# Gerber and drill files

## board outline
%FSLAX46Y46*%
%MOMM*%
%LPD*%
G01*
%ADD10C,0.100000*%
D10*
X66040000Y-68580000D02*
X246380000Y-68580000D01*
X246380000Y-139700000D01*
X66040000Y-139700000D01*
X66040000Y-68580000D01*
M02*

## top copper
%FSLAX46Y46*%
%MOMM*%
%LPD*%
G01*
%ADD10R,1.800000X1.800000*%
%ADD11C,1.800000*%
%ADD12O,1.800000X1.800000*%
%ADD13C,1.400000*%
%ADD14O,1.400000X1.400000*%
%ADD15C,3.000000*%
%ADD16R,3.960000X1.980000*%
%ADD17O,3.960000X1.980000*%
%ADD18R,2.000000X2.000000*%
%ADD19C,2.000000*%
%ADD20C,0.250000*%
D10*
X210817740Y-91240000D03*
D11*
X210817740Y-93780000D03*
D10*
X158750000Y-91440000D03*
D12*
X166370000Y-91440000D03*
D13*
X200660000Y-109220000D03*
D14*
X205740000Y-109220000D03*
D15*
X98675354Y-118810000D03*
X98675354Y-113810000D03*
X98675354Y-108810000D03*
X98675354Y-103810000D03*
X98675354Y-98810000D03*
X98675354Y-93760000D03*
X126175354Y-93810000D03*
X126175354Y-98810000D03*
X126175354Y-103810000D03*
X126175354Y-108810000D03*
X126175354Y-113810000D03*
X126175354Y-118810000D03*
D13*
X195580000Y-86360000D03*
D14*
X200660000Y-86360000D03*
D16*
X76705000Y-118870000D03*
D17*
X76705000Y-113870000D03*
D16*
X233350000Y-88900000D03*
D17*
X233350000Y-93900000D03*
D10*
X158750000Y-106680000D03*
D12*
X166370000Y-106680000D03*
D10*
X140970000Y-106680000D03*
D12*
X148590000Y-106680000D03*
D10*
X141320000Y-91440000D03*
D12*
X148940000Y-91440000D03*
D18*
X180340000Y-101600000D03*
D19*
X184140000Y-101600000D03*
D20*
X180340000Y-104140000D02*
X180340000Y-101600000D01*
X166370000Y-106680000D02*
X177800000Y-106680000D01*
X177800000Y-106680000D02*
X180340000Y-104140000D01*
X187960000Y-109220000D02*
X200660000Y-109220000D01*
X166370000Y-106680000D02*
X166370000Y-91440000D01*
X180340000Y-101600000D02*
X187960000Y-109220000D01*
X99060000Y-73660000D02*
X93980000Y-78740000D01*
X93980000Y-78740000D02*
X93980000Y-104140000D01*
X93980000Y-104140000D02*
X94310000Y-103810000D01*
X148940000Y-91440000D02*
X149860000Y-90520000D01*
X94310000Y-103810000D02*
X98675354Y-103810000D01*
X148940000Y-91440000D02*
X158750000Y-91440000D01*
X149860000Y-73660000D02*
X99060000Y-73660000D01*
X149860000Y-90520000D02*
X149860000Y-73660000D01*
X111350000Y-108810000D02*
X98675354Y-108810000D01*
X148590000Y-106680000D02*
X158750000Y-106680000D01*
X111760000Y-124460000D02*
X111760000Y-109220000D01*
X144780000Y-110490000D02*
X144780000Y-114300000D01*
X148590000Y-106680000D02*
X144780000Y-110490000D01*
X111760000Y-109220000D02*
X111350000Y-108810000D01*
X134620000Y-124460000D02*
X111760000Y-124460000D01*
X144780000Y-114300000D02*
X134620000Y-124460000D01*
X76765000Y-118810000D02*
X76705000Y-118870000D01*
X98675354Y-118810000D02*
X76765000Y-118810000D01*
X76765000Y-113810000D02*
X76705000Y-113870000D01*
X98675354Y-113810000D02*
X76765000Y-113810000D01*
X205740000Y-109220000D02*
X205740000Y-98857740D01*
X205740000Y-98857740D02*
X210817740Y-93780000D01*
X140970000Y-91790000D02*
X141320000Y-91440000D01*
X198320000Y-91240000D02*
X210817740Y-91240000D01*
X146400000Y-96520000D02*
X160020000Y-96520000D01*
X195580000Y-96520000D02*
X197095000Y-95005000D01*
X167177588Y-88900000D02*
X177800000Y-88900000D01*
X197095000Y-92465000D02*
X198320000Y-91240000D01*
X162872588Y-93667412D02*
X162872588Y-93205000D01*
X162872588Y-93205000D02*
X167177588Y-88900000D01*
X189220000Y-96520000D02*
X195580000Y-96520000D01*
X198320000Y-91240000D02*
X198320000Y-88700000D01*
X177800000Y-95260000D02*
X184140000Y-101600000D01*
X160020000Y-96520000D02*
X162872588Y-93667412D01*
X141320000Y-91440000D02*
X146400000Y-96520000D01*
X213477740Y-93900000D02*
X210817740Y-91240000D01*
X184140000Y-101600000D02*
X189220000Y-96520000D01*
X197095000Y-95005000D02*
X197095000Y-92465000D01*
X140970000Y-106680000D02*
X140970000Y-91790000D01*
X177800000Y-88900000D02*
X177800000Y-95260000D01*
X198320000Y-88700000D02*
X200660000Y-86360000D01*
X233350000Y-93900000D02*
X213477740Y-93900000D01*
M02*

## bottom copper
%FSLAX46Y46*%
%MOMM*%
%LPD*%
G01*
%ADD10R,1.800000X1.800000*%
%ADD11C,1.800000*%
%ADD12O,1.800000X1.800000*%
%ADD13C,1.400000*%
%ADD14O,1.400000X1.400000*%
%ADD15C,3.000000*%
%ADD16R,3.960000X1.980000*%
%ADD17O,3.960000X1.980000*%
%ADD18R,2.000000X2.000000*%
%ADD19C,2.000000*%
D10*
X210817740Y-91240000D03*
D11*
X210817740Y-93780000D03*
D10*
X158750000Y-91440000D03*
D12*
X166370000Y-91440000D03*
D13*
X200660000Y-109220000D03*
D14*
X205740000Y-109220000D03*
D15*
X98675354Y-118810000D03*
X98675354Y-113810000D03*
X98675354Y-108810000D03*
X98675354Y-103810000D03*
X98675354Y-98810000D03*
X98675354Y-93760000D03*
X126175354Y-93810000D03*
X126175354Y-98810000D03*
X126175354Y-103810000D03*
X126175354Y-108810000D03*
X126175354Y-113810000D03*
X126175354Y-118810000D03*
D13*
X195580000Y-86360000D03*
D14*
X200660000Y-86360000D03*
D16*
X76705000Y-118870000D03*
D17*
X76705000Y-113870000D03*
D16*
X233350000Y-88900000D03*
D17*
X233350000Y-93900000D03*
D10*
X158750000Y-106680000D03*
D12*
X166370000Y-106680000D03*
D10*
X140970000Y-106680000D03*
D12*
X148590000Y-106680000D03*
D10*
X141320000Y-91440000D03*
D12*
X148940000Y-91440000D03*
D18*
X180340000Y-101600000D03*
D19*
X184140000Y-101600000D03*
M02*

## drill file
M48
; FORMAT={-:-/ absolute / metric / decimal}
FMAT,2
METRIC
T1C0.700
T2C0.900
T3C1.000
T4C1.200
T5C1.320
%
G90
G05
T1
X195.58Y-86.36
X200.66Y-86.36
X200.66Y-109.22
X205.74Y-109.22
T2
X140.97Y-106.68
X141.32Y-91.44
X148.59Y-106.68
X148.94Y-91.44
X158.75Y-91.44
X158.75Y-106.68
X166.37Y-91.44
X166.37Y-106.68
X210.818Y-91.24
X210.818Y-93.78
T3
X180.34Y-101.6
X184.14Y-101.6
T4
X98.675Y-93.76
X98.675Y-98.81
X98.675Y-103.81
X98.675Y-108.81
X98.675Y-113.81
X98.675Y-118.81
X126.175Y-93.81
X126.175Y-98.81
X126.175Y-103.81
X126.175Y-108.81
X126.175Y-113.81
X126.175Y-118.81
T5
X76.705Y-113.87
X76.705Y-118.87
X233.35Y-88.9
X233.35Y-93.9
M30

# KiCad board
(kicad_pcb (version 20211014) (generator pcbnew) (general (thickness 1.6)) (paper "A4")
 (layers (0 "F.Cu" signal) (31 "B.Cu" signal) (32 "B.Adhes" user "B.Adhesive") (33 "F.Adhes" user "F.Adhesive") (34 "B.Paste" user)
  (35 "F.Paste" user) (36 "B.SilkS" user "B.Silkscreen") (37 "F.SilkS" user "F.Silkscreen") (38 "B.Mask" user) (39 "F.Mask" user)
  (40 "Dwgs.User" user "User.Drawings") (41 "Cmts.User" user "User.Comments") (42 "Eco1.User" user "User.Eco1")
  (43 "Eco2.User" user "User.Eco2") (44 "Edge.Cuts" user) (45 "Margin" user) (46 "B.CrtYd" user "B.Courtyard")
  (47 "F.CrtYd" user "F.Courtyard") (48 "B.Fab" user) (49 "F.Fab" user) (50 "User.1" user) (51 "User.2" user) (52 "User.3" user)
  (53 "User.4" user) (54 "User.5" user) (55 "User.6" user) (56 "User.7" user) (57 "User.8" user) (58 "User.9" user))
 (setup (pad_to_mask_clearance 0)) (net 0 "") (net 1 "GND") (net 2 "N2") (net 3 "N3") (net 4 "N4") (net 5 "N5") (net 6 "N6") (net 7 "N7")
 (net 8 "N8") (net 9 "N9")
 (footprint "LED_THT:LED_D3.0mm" (layer "F.Cu") (at 210.81774 91.24 -90)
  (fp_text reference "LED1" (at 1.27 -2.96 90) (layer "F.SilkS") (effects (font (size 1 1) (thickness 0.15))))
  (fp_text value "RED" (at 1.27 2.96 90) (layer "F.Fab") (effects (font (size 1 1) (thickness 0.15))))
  (pad "1" thru_hole rect (at 0 0 270) (size 1.8 1.8) (drill 0.9) (layers *.Cu *.Mask) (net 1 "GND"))
  (pad "2" thru_hole circle (at 2.54 0 270) (size 1.8 1.8) (drill 0.9) (layers *.Cu *.Mask) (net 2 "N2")))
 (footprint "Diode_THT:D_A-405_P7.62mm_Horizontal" (layer "F.Cu") (at 158.75 91.44)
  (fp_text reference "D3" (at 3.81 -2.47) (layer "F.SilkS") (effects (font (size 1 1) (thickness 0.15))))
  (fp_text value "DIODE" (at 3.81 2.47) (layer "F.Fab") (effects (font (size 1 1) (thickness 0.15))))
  (pad "1" thru_hole rect (at 0 0) (size 1.8 1.8) (drill 0.9) (layers *.Cu *.Mask) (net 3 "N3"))
  (pad "2" thru_hole oval (at 7.62 0) (size 1.8 1.8) (drill 0.9) (layers *.Cu *.Mask) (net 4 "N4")))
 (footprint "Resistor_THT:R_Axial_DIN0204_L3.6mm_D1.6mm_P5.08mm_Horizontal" (layer "F.Cu") (at 200.66 109.22)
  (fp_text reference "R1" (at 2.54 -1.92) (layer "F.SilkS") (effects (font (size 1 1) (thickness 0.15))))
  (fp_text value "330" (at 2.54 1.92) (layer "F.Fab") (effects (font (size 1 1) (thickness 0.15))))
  (pad "1" thru_hole circle (at 0 0) (size 1.4 1.4) (drill 0.7) (layers *.Cu *.Mask) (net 4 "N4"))
  (pad "2" thru_hole oval (at 5.08 0) (size 1.4 1.4) (drill 0.7) (layers *.Cu *.Mask) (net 2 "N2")))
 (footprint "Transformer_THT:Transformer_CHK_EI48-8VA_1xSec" (layer "F.Cu") (at 98.675354 118.81)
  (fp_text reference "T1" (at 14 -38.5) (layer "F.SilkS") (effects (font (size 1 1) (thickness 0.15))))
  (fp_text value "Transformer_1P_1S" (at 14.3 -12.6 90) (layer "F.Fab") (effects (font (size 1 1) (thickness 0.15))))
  (pad "1" thru_hole circle (at 0 0) (size 3 3) (drill 1.2) (layers *.Cu *.Mask) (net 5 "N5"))
  (pad "2" thru_hole circle (at 0 -5) (size 3 3) (drill 1.2) (layers *.Cu *.Mask) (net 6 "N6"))
  (pad "3" thru_hole circle (at 0 -10) (size 3 3) (drill 1.2) (layers *.Cu *.Mask) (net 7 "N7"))
  (pad "4" thru_hole circle (at 0 -15) (size 3 3) (drill 1.2) (layers *.Cu *.Mask) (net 3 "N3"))
  (pad "5" thru_hole circle (at 0 -20) (size 3 3) (drill 1.2) (layers *.Cu *.Mask))
  (pad "6" thru_hole circle (at 0 -25.05) (size 3 3) (drill 1.2) (layers *.Cu *.Mask))
  (pad "7" thru_hole circle (at 27.5 -25) (size 3 3) (drill 1.2) (layers *.Cu *.Mask))
  (pad "8" thru_hole circle (at 27.5 -20) (size 3 3) (drill 1.2) (layers *.Cu *.Mask))
  (pad "9" thru_hole circle (at 27.5 -15) (size 3 3) (drill 1.2) (layers *.Cu *.Mask))
  (pad "10" thru_hole circle (at 27.5 -10) (size 3 3) (drill 1.2) (layers *.Cu *.Mask))
  (pad "11" thru_hole circle (at 27.5 -5) (size 3 3) (drill 1.2) (layers *.Cu *.Mask))
  (pad "12" thru_hole circle (at 27.5 0) (size 3 3) (drill 1.2) (layers *.Cu *.Mask)))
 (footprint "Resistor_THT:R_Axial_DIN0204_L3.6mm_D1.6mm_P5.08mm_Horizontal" (layer "F.Cu") (at 195.58 86.36)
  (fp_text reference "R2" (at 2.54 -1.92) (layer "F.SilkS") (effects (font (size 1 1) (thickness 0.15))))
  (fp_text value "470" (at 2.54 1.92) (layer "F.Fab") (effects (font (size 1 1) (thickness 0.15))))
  (pad "1" thru_hole circle (at 0 0) (size 1.4 1.4) (drill 0.7) (layers *.Cu *.Mask) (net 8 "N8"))
  (pad "2" thru_hole oval (at 5.08 0) (size 1.4 1.4) (drill 0.7) (layers *.Cu *.Mask) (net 1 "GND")))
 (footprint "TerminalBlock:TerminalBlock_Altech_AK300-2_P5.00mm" (layer "F.Cu") (at 76.705 118.87 90)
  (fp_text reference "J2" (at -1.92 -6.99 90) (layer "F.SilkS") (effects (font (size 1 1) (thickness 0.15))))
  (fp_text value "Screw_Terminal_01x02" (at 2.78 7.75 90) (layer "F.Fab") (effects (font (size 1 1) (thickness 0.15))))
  (pad "1" thru_hole rect (at 0 0 90) (size 1.98 3.96) (drill 1.32) (layers *.Cu *.Mask) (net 5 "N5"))
  (pad "2" thru_hole oval (at 5 0 90) (size 1.98 3.96) (drill 1.32) (layers *.Cu *.Mask) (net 6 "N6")))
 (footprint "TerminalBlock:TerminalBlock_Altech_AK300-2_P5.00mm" (layer "F.Cu") (at 233.35 88.9 -90)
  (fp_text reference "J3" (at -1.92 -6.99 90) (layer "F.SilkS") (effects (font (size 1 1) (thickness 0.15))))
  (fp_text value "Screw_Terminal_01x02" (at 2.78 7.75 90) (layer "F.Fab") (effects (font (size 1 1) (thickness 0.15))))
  (pad "1" thru_hole rect (at 0 0 270) (size 1.98 3.96) (drill 1.32) (layers *.Cu *.Mask) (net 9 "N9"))
  (pad "2" thru_hole oval (at 5 0 270) (size 1.98 3.96) (drill 1.32) (layers *.Cu *.Mask) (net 1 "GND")))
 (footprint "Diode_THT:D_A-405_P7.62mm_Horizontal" (layer "F.Cu") (at 158.75 106.68)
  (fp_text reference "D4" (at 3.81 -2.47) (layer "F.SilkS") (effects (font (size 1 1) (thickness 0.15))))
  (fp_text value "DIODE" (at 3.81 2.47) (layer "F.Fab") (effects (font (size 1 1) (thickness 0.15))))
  (pad "1" thru_hole rect (at 0 0) (size 1.8 1.8) (drill 0.9) (layers *.Cu *.Mask) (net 7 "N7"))
  (pad "2" thru_hole oval (at 7.62 0) (size 1.8 1.8) (drill 0.9) (layers *.Cu *.Mask) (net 4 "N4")))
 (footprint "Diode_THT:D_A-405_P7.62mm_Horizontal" (layer "F.Cu") (at 140.97 106.68)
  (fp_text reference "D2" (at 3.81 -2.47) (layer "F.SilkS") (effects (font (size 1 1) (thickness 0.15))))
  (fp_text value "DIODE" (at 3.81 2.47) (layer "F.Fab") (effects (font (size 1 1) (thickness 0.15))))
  (pad "1" thru_hole rect (at 0 0) (size 1.8 1.8) (drill 0.9) (layers *.Cu *.Mask) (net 1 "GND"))
  (pad "2" thru_hole oval (at 7.62 0) (size 1.8 1.8) (drill 0.9) (layers *.Cu *.Mask) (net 7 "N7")))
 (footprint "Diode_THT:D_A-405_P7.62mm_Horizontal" (layer "F.Cu") (at 141.32 91.44)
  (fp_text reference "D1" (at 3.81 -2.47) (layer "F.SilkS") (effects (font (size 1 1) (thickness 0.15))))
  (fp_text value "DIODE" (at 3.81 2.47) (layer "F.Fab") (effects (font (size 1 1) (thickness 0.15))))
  (pad "1" thru_hole rect (at 0 0) (size 1.8 1.8) (drill 0.9) (layers *.Cu *.Mask) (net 1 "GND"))
  (pad "2" thru_hole oval (at 7.62 0) (size 1.8 1.8) (drill 0.9) (layers *.Cu *.Mask) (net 3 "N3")))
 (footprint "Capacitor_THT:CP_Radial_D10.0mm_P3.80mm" (layer "F.Cu") (at 180.34 101.6)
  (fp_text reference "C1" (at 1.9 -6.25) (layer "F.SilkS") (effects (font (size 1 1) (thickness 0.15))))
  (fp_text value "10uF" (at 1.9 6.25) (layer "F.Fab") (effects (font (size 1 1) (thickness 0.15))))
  (pad "1" thru_hole rect (at 0 0) (size 2 2) (drill 1) (layers *.Cu *.Mask) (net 4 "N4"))
  (pad "2" thru_hole circle (at 3.8 0) (size 2 2) (drill 1) (layers *.Cu *.Mask) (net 1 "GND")))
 (gr_rect (start 66.04 68.58) (end 246.38 139.7) (layer "Edge.Cuts") (width 0.1) (fill none))
 (segment (start 180.34 104.14) (end 180.34 101.6) (width 0.25) (layer "F.Cu") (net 4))
 (segment (start 166.37 106.68) (end 177.8 106.68) (width 0.25) (layer "F.Cu") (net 4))
 (segment (start 177.8 106.68) (end 180.34 104.14) (width 0.25) (layer "F.Cu") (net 4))
 (segment (start 187.96 109.22) (end 200.66 109.22) (width 0.25) (layer "F.Cu") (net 4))
 (segment (start 166.37 106.68) (end 166.37 91.44) (width 0.25) (layer "F.Cu") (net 4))
 (segment (start 180.34 101.6) (end 187.96 109.22) (width 0.25) (layer "F.Cu") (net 4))
 (segment (start 99.06 73.66) (end 93.98 78.74) (width 0.25) (layer "F.Cu") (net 3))
 (segment (start 93.98 78.74) (end 93.98 104.14) (width 0.25) (layer "F.Cu") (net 3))
 (segment (start 93.98 104.14) (end 94.31 103.81) (width 0.25) (layer "F.Cu") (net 3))
 (segment (start 148.94 91.44) (end 149.86 90.52) (width 0.25) (layer "F.Cu") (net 3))
 (segment (start 94.31 103.81) (end 98.675354 103.81) (width 0.25) (layer "F.Cu") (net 3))
 (segment (start 148.94 91.44) (end 158.75 91.44) (width 0.25) (layer "F.Cu") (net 3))
 (segment (start 149.86 73.66) (end 99.06 73.66) (width 0.25) (layer "F.Cu") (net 3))
 (segment (start 149.86 90.52) (end 149.86 73.66) (width 0.25) (layer "F.Cu") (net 3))
 (segment (start 111.35 108.81) (end 98.675354 108.81) (width 0.25) (layer "F.Cu") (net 7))
 (segment (start 148.59 106.68) (end 158.75 106.68) (width 0.25) (layer "F.Cu") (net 7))
 (segment (start 111.76 124.46) (end 111.76 109.22) (width 0.25) (layer "F.Cu") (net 7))
 (segment (start 144.78 110.49) (end 144.78 114.3) (width 0.25) (layer "F.Cu") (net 7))
 (segment (start 148.59 106.68) (end 144.78 110.49) (width 0.25) (layer "F.Cu") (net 7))
 (segment (start 111.76 109.22) (end 111.35 108.81) (width 0.25) (layer "F.Cu") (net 7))
 (segment (start 134.62 124.46) (end 111.76 124.46) (width 0.25) (layer "F.Cu") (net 7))
 (segment (start 144.78 114.3) (end 134.62 124.46) (width 0.25) (layer "F.Cu") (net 7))
 (segment (start 76.765 118.81) (end 76.705 118.87) (width 0.25) (layer "F.Cu") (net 5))
 (segment (start 98.675354 118.81) (end 76.765 118.81) (width 0.25) (layer "F.Cu") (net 5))
 (segment (start 76.765 113.81) (end 76.705 113.87) (width 0.25) (layer "F.Cu") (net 6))
 (segment (start 98.675354 113.81) (end 76.765 113.81) (width 0.25) (layer "F.Cu") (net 6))
 (segment (start 205.74 109.22) (end 205.74 98.85774) (width 0.25) (layer "F.Cu") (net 2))
 (segment (start 205.74 98.85774) (end 210.81774 93.78) (width 0.25) (layer "F.Cu") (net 2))
 (segment (start 140.97 91.79) (end 141.32 91.44) (width 0.25) (layer "F.Cu") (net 1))
 (segment (start 198.32 91.24) (end 210.81774 91.24) (width 0.25) (layer "F.Cu") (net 1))
 (segment (start 146.4 96.52) (end 160.02 96.52) (width 0.25) (layer "F.Cu") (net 1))
 (segment (start 195.58 96.52) (end 197.095 95.005) (width 0.25) (layer "F.Cu") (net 1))
 (segment (start 167.177588 88.9) (end 177.8 88.9) (width 0.25) (layer "F.Cu") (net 1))
 (segment (start 197.095 92.465) (end 198.32 91.24) (width 0.25) (layer "F.Cu") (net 1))
 (segment (start 162.872588 93.667412) (end 162.872588 93.205) (width 0.25) (layer "F.Cu") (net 1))
 (segment (start 162.872588 93.205) (end 167.177588 88.9) (width 0.25) (layer "F.Cu") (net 1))
 (segment (start 189.22 96.52) (end 195.58 96.52) (width 0.25) (layer "F.Cu") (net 1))
 (segment (start 198.32 91.24) (end 198.32 88.7) (width 0.25) (layer "F.Cu") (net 1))
 (segment (start 177.8 95.26) (end 184.14 101.6) (width 0.25) (layer "F.Cu") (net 1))
 (segment (start 160.02 96.52) (end 162.872588 93.667412) (width 0.25) (layer "F.Cu") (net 1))
 (segment (start 141.32 91.44) (end 146.4 96.52) (width 0.25) (layer "F.Cu") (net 1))
 (segment (start 213.47774 93.9) (end 210.81774 91.24) (width 0.25) (layer "F.Cu") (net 1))
 (segment (start 184.14 101.6) (end 189.22 96.52) (width 0.25) (layer "F.Cu") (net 1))
 (segment (start 197.095 95.005) (end 197.095 92.465) (width 0.25) (layer "F.Cu") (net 1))
 (segment (start 140.97 106.68) (end 140.97 91.79) (width 0.25) (layer "F.Cu") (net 1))
 (segment (start 177.8 88.9) (end 177.8 95.26) (width 0.25) (layer "F.Cu") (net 1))
 (segment (start 198.32 88.7) (end 200.66 86.36) (width 0.25) (layer "F.Cu") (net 1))
 (segment (start 233.35 93.9) (end 213.47774 93.9) (width 0.25) (layer "F.Cu") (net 1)))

